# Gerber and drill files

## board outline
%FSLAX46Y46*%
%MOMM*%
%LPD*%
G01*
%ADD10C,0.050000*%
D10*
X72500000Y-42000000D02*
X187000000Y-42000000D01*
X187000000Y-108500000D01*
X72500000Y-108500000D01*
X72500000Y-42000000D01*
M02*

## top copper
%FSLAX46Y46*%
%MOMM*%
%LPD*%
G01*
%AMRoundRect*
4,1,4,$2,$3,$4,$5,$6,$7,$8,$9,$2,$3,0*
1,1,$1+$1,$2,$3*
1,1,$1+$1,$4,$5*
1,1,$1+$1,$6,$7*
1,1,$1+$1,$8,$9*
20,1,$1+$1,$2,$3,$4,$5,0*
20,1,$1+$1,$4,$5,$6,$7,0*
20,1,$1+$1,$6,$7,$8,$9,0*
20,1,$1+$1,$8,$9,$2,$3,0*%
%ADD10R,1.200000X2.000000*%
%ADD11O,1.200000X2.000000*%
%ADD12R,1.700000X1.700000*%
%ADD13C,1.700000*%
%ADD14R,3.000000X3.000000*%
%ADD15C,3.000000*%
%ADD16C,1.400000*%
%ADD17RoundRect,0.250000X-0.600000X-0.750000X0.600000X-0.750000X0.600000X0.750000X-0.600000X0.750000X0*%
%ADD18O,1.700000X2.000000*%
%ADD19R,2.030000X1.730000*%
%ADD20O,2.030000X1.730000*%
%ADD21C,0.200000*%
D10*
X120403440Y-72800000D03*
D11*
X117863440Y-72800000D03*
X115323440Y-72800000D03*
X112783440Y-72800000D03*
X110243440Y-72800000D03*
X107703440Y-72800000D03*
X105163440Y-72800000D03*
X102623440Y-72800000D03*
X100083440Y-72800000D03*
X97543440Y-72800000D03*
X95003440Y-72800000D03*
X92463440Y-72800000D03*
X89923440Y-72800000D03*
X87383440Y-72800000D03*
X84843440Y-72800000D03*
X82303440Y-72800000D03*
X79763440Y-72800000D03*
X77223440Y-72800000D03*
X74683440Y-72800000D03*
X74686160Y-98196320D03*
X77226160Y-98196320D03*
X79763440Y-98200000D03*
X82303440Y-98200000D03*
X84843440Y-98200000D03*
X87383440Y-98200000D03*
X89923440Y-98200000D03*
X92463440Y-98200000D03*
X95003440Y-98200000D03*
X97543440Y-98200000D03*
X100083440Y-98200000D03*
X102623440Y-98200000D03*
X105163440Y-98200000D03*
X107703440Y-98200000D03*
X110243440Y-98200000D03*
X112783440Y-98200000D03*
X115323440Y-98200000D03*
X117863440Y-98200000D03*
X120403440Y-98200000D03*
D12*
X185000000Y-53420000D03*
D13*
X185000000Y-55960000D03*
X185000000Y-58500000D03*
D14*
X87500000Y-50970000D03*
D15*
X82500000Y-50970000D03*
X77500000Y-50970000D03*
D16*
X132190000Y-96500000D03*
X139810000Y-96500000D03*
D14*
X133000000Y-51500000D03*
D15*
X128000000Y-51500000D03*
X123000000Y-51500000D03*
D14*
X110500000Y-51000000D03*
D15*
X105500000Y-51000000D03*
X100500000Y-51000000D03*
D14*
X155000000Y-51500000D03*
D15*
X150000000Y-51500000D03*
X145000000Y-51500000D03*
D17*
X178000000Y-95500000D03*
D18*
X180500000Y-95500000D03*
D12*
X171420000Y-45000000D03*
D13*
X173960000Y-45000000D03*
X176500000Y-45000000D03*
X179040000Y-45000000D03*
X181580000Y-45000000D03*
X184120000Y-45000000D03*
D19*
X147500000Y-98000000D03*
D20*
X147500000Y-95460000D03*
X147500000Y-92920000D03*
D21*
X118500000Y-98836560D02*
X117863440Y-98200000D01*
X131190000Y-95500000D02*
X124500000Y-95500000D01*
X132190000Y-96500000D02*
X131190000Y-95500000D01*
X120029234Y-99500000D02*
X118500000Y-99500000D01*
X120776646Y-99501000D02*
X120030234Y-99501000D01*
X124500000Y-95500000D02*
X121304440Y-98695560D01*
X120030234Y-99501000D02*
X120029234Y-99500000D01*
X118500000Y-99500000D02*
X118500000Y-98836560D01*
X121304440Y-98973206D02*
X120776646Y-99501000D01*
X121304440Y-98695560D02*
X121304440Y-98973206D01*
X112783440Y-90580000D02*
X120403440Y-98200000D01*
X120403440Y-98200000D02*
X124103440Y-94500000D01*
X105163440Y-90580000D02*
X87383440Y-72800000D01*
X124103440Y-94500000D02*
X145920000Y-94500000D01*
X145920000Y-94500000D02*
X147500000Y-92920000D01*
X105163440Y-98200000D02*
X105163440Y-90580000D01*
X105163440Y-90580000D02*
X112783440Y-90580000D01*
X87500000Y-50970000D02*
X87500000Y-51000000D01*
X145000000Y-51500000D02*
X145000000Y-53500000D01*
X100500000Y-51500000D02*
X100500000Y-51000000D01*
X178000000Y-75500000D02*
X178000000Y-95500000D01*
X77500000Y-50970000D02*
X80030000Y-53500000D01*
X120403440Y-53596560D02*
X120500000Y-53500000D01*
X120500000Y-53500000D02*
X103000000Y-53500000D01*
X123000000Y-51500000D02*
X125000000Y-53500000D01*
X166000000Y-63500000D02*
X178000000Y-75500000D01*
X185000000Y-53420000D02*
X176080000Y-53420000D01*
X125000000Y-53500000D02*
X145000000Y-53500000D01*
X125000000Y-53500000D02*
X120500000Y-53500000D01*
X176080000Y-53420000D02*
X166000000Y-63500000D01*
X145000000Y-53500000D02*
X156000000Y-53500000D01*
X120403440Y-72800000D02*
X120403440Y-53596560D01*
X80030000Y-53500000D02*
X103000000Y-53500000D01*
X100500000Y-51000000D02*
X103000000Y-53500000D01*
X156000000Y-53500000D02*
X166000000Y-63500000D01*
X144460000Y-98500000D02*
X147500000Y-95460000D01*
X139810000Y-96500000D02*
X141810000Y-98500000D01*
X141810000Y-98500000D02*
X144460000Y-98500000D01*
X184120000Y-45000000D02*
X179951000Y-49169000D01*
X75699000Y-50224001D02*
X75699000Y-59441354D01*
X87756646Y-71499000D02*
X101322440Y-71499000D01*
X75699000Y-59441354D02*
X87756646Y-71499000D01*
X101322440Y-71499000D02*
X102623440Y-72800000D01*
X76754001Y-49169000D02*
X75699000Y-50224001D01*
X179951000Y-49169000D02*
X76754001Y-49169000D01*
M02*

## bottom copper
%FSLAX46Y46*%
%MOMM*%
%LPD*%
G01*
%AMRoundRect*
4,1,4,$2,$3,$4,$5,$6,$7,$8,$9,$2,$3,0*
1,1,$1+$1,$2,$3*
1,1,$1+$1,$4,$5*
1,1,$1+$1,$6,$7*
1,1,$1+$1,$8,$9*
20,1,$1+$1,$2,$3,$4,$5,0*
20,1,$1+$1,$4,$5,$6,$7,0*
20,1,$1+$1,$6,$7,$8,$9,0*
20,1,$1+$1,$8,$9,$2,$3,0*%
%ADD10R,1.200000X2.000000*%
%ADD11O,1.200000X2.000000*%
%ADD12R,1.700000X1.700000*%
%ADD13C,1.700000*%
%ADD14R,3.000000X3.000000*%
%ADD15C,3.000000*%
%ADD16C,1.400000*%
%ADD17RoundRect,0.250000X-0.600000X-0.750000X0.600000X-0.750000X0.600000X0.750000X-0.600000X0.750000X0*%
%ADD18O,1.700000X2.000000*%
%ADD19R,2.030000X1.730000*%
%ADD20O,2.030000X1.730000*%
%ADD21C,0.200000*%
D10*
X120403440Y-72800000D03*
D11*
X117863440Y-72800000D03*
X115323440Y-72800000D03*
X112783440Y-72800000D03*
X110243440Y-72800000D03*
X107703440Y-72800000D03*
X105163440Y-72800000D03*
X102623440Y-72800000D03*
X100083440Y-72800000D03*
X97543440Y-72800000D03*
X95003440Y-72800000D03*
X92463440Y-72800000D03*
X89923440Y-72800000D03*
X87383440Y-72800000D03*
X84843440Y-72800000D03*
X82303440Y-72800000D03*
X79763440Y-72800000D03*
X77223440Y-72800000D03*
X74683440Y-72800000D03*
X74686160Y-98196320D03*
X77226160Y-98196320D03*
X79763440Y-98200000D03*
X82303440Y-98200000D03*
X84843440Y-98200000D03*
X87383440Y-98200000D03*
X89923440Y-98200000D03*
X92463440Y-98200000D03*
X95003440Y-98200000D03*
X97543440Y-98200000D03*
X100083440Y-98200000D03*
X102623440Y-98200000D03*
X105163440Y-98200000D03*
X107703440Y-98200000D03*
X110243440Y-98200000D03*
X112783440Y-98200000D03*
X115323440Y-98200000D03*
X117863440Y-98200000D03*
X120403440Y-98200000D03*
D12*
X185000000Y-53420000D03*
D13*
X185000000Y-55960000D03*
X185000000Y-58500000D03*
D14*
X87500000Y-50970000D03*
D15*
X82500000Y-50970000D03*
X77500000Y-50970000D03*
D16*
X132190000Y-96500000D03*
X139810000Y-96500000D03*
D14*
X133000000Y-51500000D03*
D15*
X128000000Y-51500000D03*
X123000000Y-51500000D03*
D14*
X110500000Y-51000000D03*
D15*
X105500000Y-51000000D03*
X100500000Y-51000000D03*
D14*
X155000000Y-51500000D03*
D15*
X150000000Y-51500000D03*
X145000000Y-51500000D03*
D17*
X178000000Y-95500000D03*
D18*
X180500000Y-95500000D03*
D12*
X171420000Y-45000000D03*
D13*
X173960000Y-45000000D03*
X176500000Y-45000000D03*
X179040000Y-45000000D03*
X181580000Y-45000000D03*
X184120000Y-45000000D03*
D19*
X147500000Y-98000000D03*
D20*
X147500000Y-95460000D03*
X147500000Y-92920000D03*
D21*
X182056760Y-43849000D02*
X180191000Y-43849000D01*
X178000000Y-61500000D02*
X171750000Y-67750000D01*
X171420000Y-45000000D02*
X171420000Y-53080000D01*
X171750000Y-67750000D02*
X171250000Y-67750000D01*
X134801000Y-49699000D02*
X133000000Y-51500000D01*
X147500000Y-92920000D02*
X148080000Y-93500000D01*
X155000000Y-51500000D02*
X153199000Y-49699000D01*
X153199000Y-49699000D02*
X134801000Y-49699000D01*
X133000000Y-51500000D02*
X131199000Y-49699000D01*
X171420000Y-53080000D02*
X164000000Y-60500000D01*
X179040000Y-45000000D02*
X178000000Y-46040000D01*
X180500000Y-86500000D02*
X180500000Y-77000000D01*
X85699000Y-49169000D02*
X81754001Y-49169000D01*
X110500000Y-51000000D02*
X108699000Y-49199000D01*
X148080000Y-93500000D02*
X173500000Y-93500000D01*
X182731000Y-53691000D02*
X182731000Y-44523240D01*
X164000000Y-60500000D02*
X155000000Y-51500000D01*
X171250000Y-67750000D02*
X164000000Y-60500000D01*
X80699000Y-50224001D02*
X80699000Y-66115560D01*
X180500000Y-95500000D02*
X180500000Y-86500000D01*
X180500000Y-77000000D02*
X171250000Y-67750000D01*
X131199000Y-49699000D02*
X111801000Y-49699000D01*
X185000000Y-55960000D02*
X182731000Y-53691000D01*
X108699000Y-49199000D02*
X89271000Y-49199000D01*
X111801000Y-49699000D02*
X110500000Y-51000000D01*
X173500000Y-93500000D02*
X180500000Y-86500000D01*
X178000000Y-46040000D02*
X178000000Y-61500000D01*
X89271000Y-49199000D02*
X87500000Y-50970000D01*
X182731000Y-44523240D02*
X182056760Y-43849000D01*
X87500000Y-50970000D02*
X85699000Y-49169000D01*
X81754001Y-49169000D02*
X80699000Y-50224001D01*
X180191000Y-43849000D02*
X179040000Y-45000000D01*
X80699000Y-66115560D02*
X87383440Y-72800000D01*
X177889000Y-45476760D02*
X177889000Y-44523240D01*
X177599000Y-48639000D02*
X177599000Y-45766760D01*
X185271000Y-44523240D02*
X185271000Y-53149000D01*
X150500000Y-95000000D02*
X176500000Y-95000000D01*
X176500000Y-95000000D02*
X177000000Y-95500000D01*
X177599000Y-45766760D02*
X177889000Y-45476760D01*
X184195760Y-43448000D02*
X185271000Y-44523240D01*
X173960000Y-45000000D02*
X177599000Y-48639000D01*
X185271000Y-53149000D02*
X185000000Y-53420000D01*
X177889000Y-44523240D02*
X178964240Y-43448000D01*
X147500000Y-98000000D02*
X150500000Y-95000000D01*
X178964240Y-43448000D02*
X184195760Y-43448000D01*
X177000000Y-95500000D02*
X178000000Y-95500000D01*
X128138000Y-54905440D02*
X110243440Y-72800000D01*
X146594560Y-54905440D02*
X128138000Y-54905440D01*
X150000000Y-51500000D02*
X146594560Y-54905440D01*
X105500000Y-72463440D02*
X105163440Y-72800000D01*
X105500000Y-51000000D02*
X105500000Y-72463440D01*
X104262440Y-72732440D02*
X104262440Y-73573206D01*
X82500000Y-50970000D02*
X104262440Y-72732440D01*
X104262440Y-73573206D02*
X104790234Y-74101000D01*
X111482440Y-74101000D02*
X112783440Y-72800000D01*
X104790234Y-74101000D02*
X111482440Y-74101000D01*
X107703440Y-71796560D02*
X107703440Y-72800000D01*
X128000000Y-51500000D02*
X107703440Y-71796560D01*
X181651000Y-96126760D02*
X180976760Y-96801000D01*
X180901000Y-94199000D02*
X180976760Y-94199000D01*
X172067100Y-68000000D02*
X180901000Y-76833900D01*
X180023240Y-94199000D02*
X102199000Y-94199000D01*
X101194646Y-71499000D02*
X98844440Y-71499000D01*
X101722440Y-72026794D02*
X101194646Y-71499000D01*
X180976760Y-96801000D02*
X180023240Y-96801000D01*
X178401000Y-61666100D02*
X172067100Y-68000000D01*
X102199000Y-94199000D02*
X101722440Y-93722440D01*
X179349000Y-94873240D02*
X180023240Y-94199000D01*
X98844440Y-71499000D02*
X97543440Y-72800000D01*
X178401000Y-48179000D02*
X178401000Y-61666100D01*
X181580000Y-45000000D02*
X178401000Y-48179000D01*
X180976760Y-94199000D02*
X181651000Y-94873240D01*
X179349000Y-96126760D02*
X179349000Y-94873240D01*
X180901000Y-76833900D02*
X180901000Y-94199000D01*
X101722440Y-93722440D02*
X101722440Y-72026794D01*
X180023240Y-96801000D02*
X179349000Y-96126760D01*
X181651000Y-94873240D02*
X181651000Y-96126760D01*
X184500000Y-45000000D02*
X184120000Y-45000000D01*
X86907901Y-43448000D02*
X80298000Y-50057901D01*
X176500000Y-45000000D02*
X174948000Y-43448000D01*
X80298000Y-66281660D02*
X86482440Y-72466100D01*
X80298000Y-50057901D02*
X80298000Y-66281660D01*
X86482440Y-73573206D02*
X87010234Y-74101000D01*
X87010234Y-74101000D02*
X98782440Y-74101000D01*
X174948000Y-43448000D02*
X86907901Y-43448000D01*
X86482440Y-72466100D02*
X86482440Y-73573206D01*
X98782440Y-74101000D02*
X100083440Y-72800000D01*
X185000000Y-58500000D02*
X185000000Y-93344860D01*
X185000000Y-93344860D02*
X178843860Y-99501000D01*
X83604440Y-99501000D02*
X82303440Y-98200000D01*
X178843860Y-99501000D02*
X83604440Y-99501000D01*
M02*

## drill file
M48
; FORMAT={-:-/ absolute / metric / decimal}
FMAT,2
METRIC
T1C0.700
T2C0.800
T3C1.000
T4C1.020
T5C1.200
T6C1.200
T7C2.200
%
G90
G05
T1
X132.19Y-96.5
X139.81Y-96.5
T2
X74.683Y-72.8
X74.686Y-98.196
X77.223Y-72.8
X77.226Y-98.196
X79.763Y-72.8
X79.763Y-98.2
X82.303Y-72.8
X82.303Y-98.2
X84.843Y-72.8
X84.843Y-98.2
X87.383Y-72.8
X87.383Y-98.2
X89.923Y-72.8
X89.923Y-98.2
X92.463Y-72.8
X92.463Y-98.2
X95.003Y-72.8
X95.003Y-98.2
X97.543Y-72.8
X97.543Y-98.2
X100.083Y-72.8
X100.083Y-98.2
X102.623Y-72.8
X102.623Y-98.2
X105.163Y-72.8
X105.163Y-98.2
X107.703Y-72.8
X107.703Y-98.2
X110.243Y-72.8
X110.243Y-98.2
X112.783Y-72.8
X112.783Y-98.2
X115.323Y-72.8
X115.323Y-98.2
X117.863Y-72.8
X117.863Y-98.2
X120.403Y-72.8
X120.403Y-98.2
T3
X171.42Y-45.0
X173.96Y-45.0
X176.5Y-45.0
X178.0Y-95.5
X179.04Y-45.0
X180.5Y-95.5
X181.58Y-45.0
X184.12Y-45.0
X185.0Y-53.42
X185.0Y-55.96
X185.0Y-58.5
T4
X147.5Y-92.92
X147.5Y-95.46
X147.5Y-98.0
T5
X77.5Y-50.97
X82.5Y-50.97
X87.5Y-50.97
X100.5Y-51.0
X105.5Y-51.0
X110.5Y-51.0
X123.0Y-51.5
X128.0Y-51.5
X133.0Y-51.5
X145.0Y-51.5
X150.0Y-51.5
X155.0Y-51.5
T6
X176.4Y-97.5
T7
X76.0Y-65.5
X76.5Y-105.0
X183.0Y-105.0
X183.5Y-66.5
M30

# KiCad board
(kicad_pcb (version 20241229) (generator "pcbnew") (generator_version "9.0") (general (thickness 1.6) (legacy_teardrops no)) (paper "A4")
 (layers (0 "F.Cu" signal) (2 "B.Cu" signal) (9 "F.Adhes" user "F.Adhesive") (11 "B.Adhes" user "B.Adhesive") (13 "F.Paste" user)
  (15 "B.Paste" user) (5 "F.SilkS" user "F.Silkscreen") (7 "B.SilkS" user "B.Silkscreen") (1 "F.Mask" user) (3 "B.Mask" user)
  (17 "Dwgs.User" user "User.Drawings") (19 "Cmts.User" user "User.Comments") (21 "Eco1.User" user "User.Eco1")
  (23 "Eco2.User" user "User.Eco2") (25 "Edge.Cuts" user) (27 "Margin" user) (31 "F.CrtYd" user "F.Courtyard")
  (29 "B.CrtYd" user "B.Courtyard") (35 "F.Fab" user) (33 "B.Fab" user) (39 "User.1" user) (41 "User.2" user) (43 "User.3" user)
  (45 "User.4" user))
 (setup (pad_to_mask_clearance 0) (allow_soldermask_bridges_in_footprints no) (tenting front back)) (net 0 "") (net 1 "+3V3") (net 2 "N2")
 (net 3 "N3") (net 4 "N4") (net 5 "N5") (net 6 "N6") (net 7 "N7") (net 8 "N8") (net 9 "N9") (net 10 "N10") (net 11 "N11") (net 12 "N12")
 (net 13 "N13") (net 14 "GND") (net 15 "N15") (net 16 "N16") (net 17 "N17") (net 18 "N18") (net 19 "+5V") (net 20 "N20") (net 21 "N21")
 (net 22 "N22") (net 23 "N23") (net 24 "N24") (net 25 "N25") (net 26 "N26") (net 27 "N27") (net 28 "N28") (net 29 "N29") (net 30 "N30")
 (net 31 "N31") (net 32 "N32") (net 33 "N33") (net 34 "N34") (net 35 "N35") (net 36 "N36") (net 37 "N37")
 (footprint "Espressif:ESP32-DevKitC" (layer "F.Cu") (at 120.40344 72.8 -90)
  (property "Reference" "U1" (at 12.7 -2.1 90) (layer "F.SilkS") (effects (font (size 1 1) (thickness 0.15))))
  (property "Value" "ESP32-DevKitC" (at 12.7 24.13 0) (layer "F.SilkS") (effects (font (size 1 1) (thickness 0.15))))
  (pad "1" thru_hole rect (at 0 0 180) (size 1.2 2) (drill 0.8) (layers "*.Cu" "*.Mask") (remove_unused_layers no) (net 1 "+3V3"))
  (pad "2" thru_hole oval (at 0 2.54 180) (size 1.2 2) (drill 0.8) (layers "*.Cu" "*.Mask") (remove_unused_layers no) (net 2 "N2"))
  (pad "3" thru_hole oval (at 0 5.08 180) (size 1.2 2) (drill 0.8) (layers "*.Cu" "*.Mask") (remove_unused_layers no) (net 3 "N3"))
  (pad "4" thru_hole oval (at 0 7.62 180) (size 1.2 2) (drill 0.8) (layers "*.Cu" "*.Mask") (remove_unused_layers no) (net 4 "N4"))
  (pad "5" thru_hole oval (at 0 10.16 180) (size 1.2 2) (drill 0.8) (layers "*.Cu" "*.Mask") (remove_unused_layers no) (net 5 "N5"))
  (pad "6" thru_hole oval (at 0 12.7 180) (size 1.2 2) (drill 0.8) (layers "*.Cu" "*.Mask") (remove_unused_layers no) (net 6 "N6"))
  (pad "7" thru_hole oval (at 0 15.24 180) (size 1.2 2) (drill 0.8) (layers "*.Cu" "*.Mask") (remove_unused_layers no) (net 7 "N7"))
  (pad "8" thru_hole oval (at 0 17.78 180) (size 1.2 2) (drill 0.8) (layers "*.Cu" "*.Mask") (remove_unused_layers no) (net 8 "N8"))
  (pad "9" thru_hole oval (at 0 20.32 180) (size 1.2 2) (drill 0.8) (layers "*.Cu" "*.Mask") (remove_unused_layers no) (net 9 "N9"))
  (pad "10" thru_hole oval (at 0 22.86 180) (size 1.2 2) (drill 0.8) (layers "*.Cu" "*.Mask") (remove_unused_layers no) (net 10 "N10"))
  (pad "11" thru_hole oval (at 0 25.4 180) (size 1.2 2) (drill 0.8) (layers "*.Cu" "*.Mask") (remove_unused_layers no) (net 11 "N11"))
  (pad "12" thru_hole oval (at 0 27.94 180) (size 1.2 2) (drill 0.8) (layers "*.Cu" "*.Mask") (remove_unused_layers no) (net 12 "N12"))
  (pad "13" thru_hole oval (at 0 30.48 180) (size 1.2 2) (drill 0.8) (layers "*.Cu" "*.Mask") (remove_unused_layers no) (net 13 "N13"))
  (pad "14" thru_hole oval (at 0 33.02 180) (size 1.2 2) (drill 0.8) (layers "*.Cu" "*.Mask") (remove_unused_layers no) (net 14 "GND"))
  (pad "15" thru_hole oval (at 0 35.56 180) (size 1.2 2) (drill 0.8) (layers "*.Cu" "*.Mask") (remove_unused_layers no) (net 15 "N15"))
  (pad "16" thru_hole oval (at 0 38.1 180) (size 1.2 2) (drill 0.8) (layers "*.Cu" "*.Mask") (remove_unused_layers no) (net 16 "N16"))
  (pad "17" thru_hole oval (at 0 40.64 180) (size 1.2 2) (drill 0.8) (layers "*.Cu" "*.Mask") (remove_unused_layers no) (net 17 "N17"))
  (pad "18" thru_hole oval (at 0 43.18 180) (size 1.2 2) (drill 0.8) (layers "*.Cu" "*.Mask") (remove_unused_layers no) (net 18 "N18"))
  (pad "19" thru_hole oval (at 0 45.72 180) (size 1.2 2) (drill 0.8) (layers "*.Cu" "*.Mask") (remove_unused_layers no) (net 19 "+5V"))
  (pad "20" thru_hole oval (at 25.39632 45.71728 180) (size 1.2 2) (drill 0.8) (layers "*.Cu" "*.Mask") (remove_unused_layers no)
   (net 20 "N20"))
  (pad "21" thru_hole oval (at 25.39632 43.17728 180) (size 1.2 2) (drill 0.8) (layers "*.Cu" "*.Mask") (remove_unused_layers no)
   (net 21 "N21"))
  (pad "22" thru_hole oval (at 25.4 40.64 180) (size 1.2 2) (drill 0.8) (layers "*.Cu" "*.Mask") (remove_unused_layers no) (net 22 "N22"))
  (pad "23" thru_hole oval (at 25.4 38.1 180) (size 1.2 2) (drill 0.8) (layers "*.Cu" "*.Mask") (remove_unused_layers no) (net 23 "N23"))
  (pad "24" thru_hole oval (at 25.4 35.56 180) (size 1.2 2) (drill 0.8) (layers "*.Cu" "*.Mask") (remove_unused_layers no) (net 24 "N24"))
  (pad "25" thru_hole oval (at 25.4 33.02 180) (size 1.2 2) (drill 0.8) (layers "*.Cu" "*.Mask") (remove_unused_layers no) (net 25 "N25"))
  (pad "26" thru_hole oval (at 25.4 30.48 180) (size 1.2 2) (drill 0.8) (layers "*.Cu" "*.Mask") (remove_unused_layers no) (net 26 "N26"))
  (pad "27" thru_hole oval (at 25.4 27.94 180) (size 1.2 2) (drill 0.8) (layers "*.Cu" "*.Mask") (remove_unused_layers no) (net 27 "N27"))
  (pad "28" thru_hole oval (at 25.4 25.4 180) (size 1.2 2) (drill 0.8) (layers "*.Cu" "*.Mask") (remove_unused_layers no) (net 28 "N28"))
  (pad "29" thru_hole oval (at 25.4 22.86 180) (size 1.2 2) (drill 0.8) (layers "*.Cu" "*.Mask") (remove_unused_layers no) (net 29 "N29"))
  (pad "30" thru_hole oval (at 25.4 20.32 180) (size 1.2 2) (drill 0.8) (layers "*.Cu" "*.Mask") (remove_unused_layers no) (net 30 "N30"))
  (pad "31" thru_hole oval (at 25.4 17.78 180) (size 1.2 2) (drill 0.8) (layers "*.Cu" "*.Mask") (remove_unused_layers no) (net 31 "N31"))
  (pad "32" thru_hole oval (at 25.4 15.24 180) (size 1.2 2) (drill 0.8) (layers "*.Cu" "*.Mask") (remove_unused_layers no) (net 14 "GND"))
  (pad "33" thru_hole oval (at 25.4 12.7 180) (size 1.2 2) (drill 0.8) (layers "*.Cu" "*.Mask") (remove_unused_layers no) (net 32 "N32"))
  (pad "34" thru_hole oval (at 25.4 10.16 180) (size 1.2 2) (drill 0.8) (layers "*.Cu" "*.Mask") (remove_unused_layers no) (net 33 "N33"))
  (pad "35" thru_hole oval (at 25.4 7.62 180) (size 1.2 2) (drill 0.8) (layers "*.Cu" "*.Mask") (remove_unused_layers no) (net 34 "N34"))
  (pad "36" thru_hole oval (at 25.4 5.08 180) (size 1.2 2) (drill 0.8) (layers "*.Cu" "*.Mask") (remove_unused_layers no) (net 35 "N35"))
  (pad "37" thru_hole oval (at 25.4 2.54 180) (size 1.2 2) (drill 0.8) (layers "*.Cu" "*.Mask") (remove_unused_layers no) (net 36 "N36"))
  (pad "38" thru_hole oval (at 25.4 0 180) (size 1.2 2) (drill 0.8) (layers "*.Cu" "*.Mask") (remove_unused_layers no) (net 14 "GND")))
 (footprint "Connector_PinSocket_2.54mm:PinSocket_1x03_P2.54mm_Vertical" (layer "F.Cu") (at 185 53.42)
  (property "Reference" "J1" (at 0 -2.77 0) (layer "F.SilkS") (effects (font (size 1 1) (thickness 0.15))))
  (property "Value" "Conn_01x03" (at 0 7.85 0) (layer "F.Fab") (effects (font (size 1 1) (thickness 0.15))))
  (pad "1" thru_hole rect (at 0 0) (size 1.7 1.7) (drill 1) (layers "*.Cu" "*.Mask") (remove_unused_layers no) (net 1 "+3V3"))
  (pad "2" thru_hole circle (at 0 2.54) (size 1.7 1.7) (drill 1) (layers "*.Cu" "*.Mask") (remove_unused_layers no) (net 14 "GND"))
  (pad "3" thru_hole circle (at 0 5.08) (size 1.7 1.7) (drill 1) (layers "*.Cu" "*.Mask") (remove_unused_layers no) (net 23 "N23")))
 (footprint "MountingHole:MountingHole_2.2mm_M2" (layer "F.Cu") (at 76.5 105)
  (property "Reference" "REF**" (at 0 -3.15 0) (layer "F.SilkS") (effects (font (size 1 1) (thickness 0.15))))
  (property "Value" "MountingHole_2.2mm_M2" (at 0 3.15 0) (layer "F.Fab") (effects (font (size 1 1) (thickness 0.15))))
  (pad "" np_thru_hole circle (at 0 0) (size 2.2 2.2) (drill 2.2) (layers "*.Cu" "*.Mask")))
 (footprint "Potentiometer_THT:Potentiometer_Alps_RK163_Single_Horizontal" (layer "F.Cu") (at 87.5 50.97 -90)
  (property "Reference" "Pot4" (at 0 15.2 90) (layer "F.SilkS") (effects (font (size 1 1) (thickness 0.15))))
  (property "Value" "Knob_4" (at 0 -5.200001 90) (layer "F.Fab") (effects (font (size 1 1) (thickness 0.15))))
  (pad "1" thru_hole rect (at 0 0 90) (size 3 3) (drill 1.2) (layers "*.Cu" "*.Mask") (remove_unused_layers no) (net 14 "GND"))
  (pad "2" thru_hole circle (at 0 5 90) (size 3 3) (drill 1.2) (layers "*.Cu" "*.Mask") (remove_unused_layers no) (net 4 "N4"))
  (pad "3" thru_hole circle (at 0 10 90) (size 3 3) (drill 1.2) (layers "*.Cu" "*.Mask") (remove_unused_layers no) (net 1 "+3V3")))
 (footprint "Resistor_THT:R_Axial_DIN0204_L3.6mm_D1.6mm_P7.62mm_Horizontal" (layer "F.Cu") (at 132.19 96.5)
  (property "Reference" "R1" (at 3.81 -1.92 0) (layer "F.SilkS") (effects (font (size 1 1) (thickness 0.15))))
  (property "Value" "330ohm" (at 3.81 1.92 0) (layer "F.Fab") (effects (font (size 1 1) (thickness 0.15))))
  (pad "1" thru_hole circle (at 0 0) (size 1.4 1.4) (drill 0.7) (layers "*.Cu" "*.Mask") (remove_unused_layers no) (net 36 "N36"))
  (pad "2" thru_hole circle (at 7.62 0) (size 1.4 1.4) (drill 0.7) (layers "*.Cu" "*.Mask") (remove_unused_layers no) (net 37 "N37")))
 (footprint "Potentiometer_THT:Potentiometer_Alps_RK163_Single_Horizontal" (layer "F.Cu") (at 133 51.5 -90)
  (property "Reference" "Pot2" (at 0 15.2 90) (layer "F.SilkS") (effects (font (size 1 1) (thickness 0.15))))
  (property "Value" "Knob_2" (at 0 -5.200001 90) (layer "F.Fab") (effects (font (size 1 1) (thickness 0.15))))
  (pad "1" thru_hole rect (at 0 0 90) (size 3 3) (drill 1.2) (layers "*.Cu" "*.Mask") (remove_unused_layers no) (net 14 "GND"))
  (pad "2" thru_hole circle (at 0 5 90) (size 3 3) (drill 1.2) (layers "*.Cu" "*.Mask") (remove_unused_layers no) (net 6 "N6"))
  (pad "3" thru_hole circle (at 0 10 90) (size 3 3) (drill 1.2) (layers "*.Cu" "*.Mask") (remove_unused_layers no) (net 1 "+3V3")))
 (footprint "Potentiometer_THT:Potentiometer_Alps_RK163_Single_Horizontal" (layer "F.Cu") (at 110.5 51 -90)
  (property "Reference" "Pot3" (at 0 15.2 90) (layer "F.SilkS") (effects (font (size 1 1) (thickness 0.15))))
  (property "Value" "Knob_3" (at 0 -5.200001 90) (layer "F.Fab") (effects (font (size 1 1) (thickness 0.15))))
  (pad "1" thru_hole rect (at 0 0 90) (size 3 3) (drill 1.2) (layers "*.Cu" "*.Mask") (remove_unused_layers no) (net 14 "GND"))
  (pad "2" thru_hole circle (at 0 5 90) (size 3 3) (drill 1.2) (layers "*.Cu" "*.Mask") (remove_unused_layers no) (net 7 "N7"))
  (pad "3" thru_hole circle (at 0 10 90) (size 3 3) (drill 1.2) (layers "*.Cu" "*.Mask") (remove_unused_layers no) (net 1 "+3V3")))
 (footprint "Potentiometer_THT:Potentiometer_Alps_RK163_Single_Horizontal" (layer "F.Cu") (at 155 51.5 -90)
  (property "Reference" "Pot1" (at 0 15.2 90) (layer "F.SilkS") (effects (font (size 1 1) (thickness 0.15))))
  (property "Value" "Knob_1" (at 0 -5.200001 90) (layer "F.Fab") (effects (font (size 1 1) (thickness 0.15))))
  (pad "1" thru_hole rect (at 0 0 90) (size 3 3) (drill 1.2) (layers "*.Cu" "*.Mask") (remove_unused_layers no) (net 14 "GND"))
  (pad "2" thru_hole circle (at 0 5 90) (size 3 3) (drill 1.2) (layers "*.Cu" "*.Mask") (remove_unused_layers no) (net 5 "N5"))
  (pad "3" thru_hole circle (at 0 10 90) (size 3 3) (drill 1.2) (layers "*.Cu" "*.Mask") (remove_unused_layers no) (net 1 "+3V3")))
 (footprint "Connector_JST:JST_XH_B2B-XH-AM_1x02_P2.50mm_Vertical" (layer "F.Cu") (at 178 95.5)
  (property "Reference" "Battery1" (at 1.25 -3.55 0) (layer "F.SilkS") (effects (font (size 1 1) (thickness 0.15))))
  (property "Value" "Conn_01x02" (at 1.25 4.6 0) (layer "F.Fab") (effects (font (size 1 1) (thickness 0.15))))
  (pad "" np_thru_hole circle (at -1.6 2) (size 1.2 1.2) (drill 1.2) (layers "*.Cu" "*.Mask"))
  (pad "1" thru_hole roundrect (at 0 0) (size 1.7 2) (drill 1) (layers "*.Cu" "*.Mask") (remove_unused_layers no)
   (roundrect_rratio 0.147059) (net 1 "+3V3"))
  (pad "2" thru_hole oval (at 2.5 0) (size 1.7 2) (drill 1) (layers "*.Cu" "*.Mask") (remove_unused_layers no) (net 14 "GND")))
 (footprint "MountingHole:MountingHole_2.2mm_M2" (layer "F.Cu") (at 76 65.5)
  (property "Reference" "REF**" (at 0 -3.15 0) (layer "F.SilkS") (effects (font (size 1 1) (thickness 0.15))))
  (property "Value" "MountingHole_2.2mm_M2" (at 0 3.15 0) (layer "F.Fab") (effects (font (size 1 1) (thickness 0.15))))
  (pad "" np_thru_hole circle (at 0 0) (size 2.2 2.2) (drill 2.2) (layers "*.Cu" "*.Mask")))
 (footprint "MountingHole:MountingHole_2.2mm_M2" (layer "F.Cu") (at 183.5 66.5)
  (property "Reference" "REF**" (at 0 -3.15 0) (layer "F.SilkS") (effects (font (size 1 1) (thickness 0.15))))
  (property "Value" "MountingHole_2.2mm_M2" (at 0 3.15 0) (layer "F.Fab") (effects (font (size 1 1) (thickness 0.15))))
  (pad "" np_thru_hole circle (at 0 0) (size 2.2 2.2) (drill 2.2) (layers "*.Cu" "*.Mask")))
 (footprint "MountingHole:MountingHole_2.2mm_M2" (layer "F.Cu") (at 183 105)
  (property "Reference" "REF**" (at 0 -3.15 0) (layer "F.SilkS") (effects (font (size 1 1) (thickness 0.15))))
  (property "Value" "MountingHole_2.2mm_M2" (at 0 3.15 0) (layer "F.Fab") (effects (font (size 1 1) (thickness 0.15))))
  (pad "" np_thru_hole circle (at 0 0) (size 2.2 2.2) (drill 2.2) (layers "*.Cu" "*.Mask")))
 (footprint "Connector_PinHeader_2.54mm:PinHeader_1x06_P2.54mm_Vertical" (layer "B.Cu") (at 171.42 45 -90)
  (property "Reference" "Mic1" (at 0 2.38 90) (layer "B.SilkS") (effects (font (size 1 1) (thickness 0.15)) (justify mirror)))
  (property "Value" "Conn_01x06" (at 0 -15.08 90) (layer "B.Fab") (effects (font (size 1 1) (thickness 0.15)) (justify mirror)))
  (pad "1" thru_hole rect (at 0 0 270) (size 1.7 1.7) (drill 1) (layers "*.Cu" "*.Mask") (remove_unused_layers no) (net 14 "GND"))
  (pad "2" thru_hole circle (at 0 -2.54 270) (size 1.7 1.7) (drill 1) (layers "*.Cu" "*.Mask") (remove_unused_layers no) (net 1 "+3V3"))
  (pad "3" thru_hole circle (at 0 -5.08 270) (size 1.7 1.7) (drill 1) (layers "*.Cu" "*.Mask") (remove_unused_layers no) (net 9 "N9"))
  (pad "4" thru_hole circle (at 0 -7.62 270) (size 1.7 1.7) (drill 1) (layers "*.Cu" "*.Mask") (remove_unused_layers no) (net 14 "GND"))
  (pad "5" thru_hole circle (at 0 -10.16 270) (size 1.7 1.7) (drill 1) (layers "*.Cu" "*.Mask") (remove_unused_layers no) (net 10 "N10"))
  (pad "6" thru_hole circle (at 0 -12.7 270) (size 1.7 1.7) (drill 1) (layers "*.Cu" "*.Mask") (remove_unused_layers no) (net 8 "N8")))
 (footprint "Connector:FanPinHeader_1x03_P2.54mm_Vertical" (layer "B.Cu") (at 147.5 98 90)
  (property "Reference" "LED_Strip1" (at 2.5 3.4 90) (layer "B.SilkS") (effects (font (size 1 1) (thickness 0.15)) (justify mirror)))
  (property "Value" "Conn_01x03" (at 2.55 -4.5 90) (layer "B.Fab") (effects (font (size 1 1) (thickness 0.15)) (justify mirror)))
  (pad "1" thru_hole rect (at 0 0) (size 2.03 1.73) (drill 1.02) (layers "*.Cu" "*.Mask") (remove_unused_layers no) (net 1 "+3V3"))
  (pad "2" thru_hole oval (at 2.54 0) (size 2.03 1.73) (drill 1.02) (layers "*.Cu" "*.Mask") (remove_unused_layers no) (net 37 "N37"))
  (pad "3" thru_hole oval (at 5.08 0) (size 2.03 1.73) (drill 1.02) (layers "*.Cu" "*.Mask") (remove_unused_layers no) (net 14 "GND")))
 (gr_rect (start 72.5 42) (end 187 108.5) (stroke (width 0.05) (type default)) (fill no) (layer "Edge.Cuts"))
 (segment (start 118.5 98.83656) (end 117.86344 98.2) (width 0.2) (layer "F.Cu") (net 36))
 (segment (start 131.19 95.5) (end 124.5 95.5) (width 0.2) (layer "F.Cu") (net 36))
 (segment (start 132.19 96.5) (end 131.19 95.5) (width 0.2) (layer "F.Cu") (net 36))
 (segment (start 120.029234 99.5) (end 118.5 99.5) (width 0.2) (layer "F.Cu") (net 36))
 (segment (start 120.776646 99.501) (end 120.030234 99.501) (width 0.2) (layer "F.Cu") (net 36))
 (segment (start 124.5 95.5) (end 121.30444 98.69556) (width 0.2) (layer "F.Cu") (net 36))
 (segment (start 120.030234 99.501) (end 120.029234 99.5) (width 0.2) (layer "F.Cu") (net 36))
 (segment (start 118.5 99.5) (end 118.5 98.83656) (width 0.2) (layer "F.Cu") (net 36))
 (segment (start 121.30444 98.973206) (end 120.776646 99.501) (width 0.2) (layer "F.Cu") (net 36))
 (segment (start 121.30444 98.69556) (end 121.30444 98.973206) (width 0.2) (layer "F.Cu") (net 36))
 (segment (start 112.78344 90.58) (end 120.40344 98.2) (width 0.2) (layer "F.Cu") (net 14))
 (segment (start 120.40344 98.2) (end 124.10344 94.5) (width 0.2) (layer "F.Cu") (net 14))
 (segment (start 105.16344 90.58) (end 87.38344 72.8) (width 0.2) (layer "F.Cu") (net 14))
 (segment (start 124.10344 94.5) (end 145.92 94.5) (width 0.2) (layer "F.Cu") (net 14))
 (segment (start 145.92 94.5) (end 147.5 92.92) (width 0.2) (layer "F.Cu") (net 14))
 (segment (start 105.16344 98.2) (end 105.16344 90.58) (width 0.2) (layer "F.Cu") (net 14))
 (segment (start 105.16344 90.58) (end 112.78344 90.58) (width 0.2) (layer "F.Cu") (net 14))
 (segment (start 87.5 50.97) (end 87.5 51) (width 0.2) (layer "F.Cu") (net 14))
 (segment (start 182.05676 43.849) (end 180.191 43.849) (width 0.2) (layer "B.Cu") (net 14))
 (segment (start 178 61.5) (end 171.75 67.75) (width 0.2) (layer "B.Cu") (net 14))
 (segment (start 171.42 45) (end 171.42 53.08) (width 0.2) (layer "B.Cu") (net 14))
 (segment (start 171.75 67.75) (end 171.25 67.75) (width 0.2) (layer "B.Cu") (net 14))
 (segment (start 134.801 49.699) (end 133 51.5) (width 0.2) (layer "B.Cu") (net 14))
 (segment (start 147.5 92.92) (end 148.08 93.5) (width 0.2) (layer "B.Cu") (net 14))
 (segment (start 155 51.5) (end 153.199 49.699) (width 0.2) (layer "B.Cu") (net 14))
 (segment (start 153.199 49.699) (end 134.801 49.699) (width 0.2) (layer "B.Cu") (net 14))
 (segment (start 133 51.5) (end 131.199 49.699) (width 0.2) (layer "B.Cu") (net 14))
 (segment (start 171.42 53.08) (end 164 60.5) (width 0.2) (layer "B.Cu") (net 14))
 (segment (start 179.04 45) (end 178 46.04) (width 0.2) (layer "B.Cu") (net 14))
 (segment (start 180.5 86.5) (end 180.5 77) (width 0.2) (layer "B.Cu") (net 14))
 (segment (start 85.699 49.169) (end 81.754001 49.169) (width 0.2) (layer "B.Cu") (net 14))
 (segment (start 110.5 51) (end 108.699 49.199) (width 0.2) (layer "B.Cu") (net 14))
 (segment (start 148.08 93.5) (end 173.5 93.5) (width 0.2) (layer "B.Cu") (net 14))
 (segment (start 182.731 53.691) (end 182.731 44.52324) (width 0.2) (layer "B.Cu") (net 14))
 (segment (start 164 60.5) (end 155 51.5) (width 0.2) (layer "B.Cu") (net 14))
 (segment (start 171.25 67.75) (end 164 60.5) (width 0.2) (layer "B.Cu") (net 14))
 (segment (start 80.699 50.224001) (end 80.699 66.11556) (width 0.2) (layer "B.Cu") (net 14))
 (segment (start 180.5 95.5) (end 180.5 86.5) (width 0.2) (layer "B.Cu") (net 14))
 (segment (start 180.5 77) (end 171.25 67.75) (width 0.2) (layer "B.Cu") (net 14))
 (segment (start 131.199 49.699) (end 111.801 49.699) (width 0.2) (layer "B.Cu") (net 14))
 (segment (start 185 55.96) (end 182.731 53.691) (width 0.2) (layer "B.Cu") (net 14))
 (segment (start 108.699 49.199) (end 89.271 49.199) (width 0.2) (layer "B.Cu") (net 14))
 (segment (start 111.801 49.699) (end 110.5 51) (width 0.2) (layer "B.Cu") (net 14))
 (segment (start 173.5 93.5) (end 180.5 86.5) (width 0.2) (layer "B.Cu") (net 14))
 (segment (start 178 46.04) (end 178 61.5) (width 0.2) (layer "B.Cu") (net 14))
 (segment (start 89.271 49.199) (end 87.5 50.97) (width 0.2) (layer "B.Cu") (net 14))
 (segment (start 182.731 44.52324) (end 182.05676 43.849) (width 0.2) (layer "B.Cu") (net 14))
 (segment (start 87.5 50.97) (end 85.699 49.169) (width 0.2) (layer "B.Cu") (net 14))
 (segment (start 81.754001 49.169) (end 80.699 50.224001) (width 0.2) (layer "B.Cu") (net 14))
 (segment (start 180.191 43.849) (end 179.04 45) (width 0.2) (layer "B.Cu") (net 14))
 (segment (start 80.699 66.11556) (end 87.38344 72.8) (width 0.2) (layer "B.Cu") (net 14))
 (segment (start 145 51.5) (end 145 53.5) (width 0.2) (layer "F.Cu") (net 1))
 (segment (start 100.5 51.5) (end 100.5 51) (width 0.2) (layer "F.Cu") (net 1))
 (segment (start 178 75.5) (end 178 95.5) (width 0.2) (layer "F.Cu") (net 1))
 (segment (start 77.5 50.97) (end 80.03 53.5) (width 0.2) (layer "F.Cu") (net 1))
 (segment (start 120.40344 53.59656) (end 120.5 53.5) (width 0.2) (layer "F.Cu") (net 1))
 (segment (start 120.5 53.5) (end 103 53.5) (width 0.2) (layer "F.Cu") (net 1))
 (segment (start 123 51.5) (end 125 53.5) (width 0.2) (layer "F.Cu") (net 1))
 (segment (start 166 63.5) (end 178 75.5) (width 0.2) (layer "F.Cu") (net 1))
 (segment (start 185 53.42) (end 176.08 53.42) (width 0.2) (layer "F.Cu") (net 1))
 (segment (start 125 53.5) (end 145 53.5) (width 0.2) (layer "F.Cu") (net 1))
 (segment (start 125 53.5) (end 120.5 53.5) (width 0.2) (layer "F.Cu") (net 1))
 (segment (start 176.08 53.42) (end 166 63.5) (width 0.2) (layer "F.Cu") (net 1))
 (segment (start 145 53.5) (end 156 53.5) (width 0.2) (layer "F.Cu") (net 1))
 (segment (start 120.40344 72.8) (end 120.40344 53.59656) (width 0.2) (layer "F.Cu") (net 1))
 (segment (start 80.03 53.5) (end 103 53.5) (width 0.2) (layer "F.Cu") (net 1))
 (segment (start 100.5 51) (end 103 53.5) (width 0.2) (layer "F.Cu") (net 1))
 (segment (start 156 53.5) (end 166 63.5) (width 0.2) (layer "F.Cu") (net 1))
 (segment (start 177.889 45.47676) (end 177.889 44.52324) (width 0.2) (layer "B.Cu") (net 1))
 (segment (start 177.599 48.639) (end 177.599 45.76676) (width 0.2) (layer "B.Cu") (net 1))
 (segment (start 185.271 44.52324) (end 185.271 53.149) (width 0.2) (layer "B.Cu") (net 1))
 (segment (start 150.5 95) (end 176.5 95) (width 0.2) (layer "B.Cu") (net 1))
 (segment (start 176.5 95) (end 177 95.5) (width 0.2) (layer "B.Cu") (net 1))
 (segment (start 177.599 45.76676) (end 177.889 45.47676) (width 0.2) (layer "B.Cu") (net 1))
 (segment (start 184.19576 43.448) (end 185.271 44.52324) (width 0.2) (layer "B.Cu") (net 1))
 (segment (start 173.96 45) (end 177.599 48.639) (width 0.2) (layer "B.Cu") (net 1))
 (segment (start 185.271 53.149) (end 185 53.42) (width 0.2) (layer "B.Cu") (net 1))
 (segment (start 177.889 44.52324) (end 178.96424 43.448) (width 0.2) (layer "B.Cu") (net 1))
 (segment (start 147.5 98) (end 150.5 95) (width 0.2) (layer "B.Cu") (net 1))
 (segment (start 178.96424 43.448) (end 184.19576 43.448) (width 0.2) (layer "B.Cu") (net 1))
 (segment (start 177 95.5) (end 178 95.5) (width 0.2) (layer "B.Cu") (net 1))
 (segment (start 128.138 54.90544) (end 110.24344 72.8) (width 0.2) (layer "B.Cu") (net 5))
 (segment (start 146.59456 54.90544) (end 128.138 54.90544) (width 0.2) (layer "B.Cu") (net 5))
 (segment (start 150 51.5) (end 146.59456 54.90544) (width 0.2) (layer "B.Cu") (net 5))
 (segment (start 105.5 72.46344) (end 105.16344 72.8) (width 0.2) (layer "B.Cu") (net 7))
 (segment (start 105.5 51) (end 105.5 72.46344) (width 0.2) (layer "B.Cu") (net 7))
 (segment (start 104.26244 72.73244) (end 104.26244 73.573206) (width 0.2) (layer "B.Cu") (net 4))
 (segment (start 82.5 50.97) (end 104.26244 72.73244) (width 0.2) (layer "B.Cu") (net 4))
 (segment (start 104.26244 73.573206) (end 104.790234 74.101) (width 0.2) (layer "B.Cu") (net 4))
 (segment (start 111.48244 74.101) (end 112.78344 72.8) (width 0.2) (layer "B.Cu") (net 4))
 (segment (start 104.790234 74.101) (end 111.48244 74.101) (width 0.2) (layer "B.Cu") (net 4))
 (segment (start 107.70344 71.79656) (end 107.70344 72.8) (width 0.2) (layer "B.Cu") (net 6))
 (segment (start 128 51.5) (end 107.70344 71.79656) (width 0.2) (layer "B.Cu") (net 6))
 (segment (start 144.46 98.5) (end 147.5 95.46) (width 0.2) (layer "F.Cu") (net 37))
 (segment (start 139.81 96.5) (end 141.81 98.5) (width 0.2) (layer "F.Cu") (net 37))
 (segment (start 141.81 98.5) (end 144.46 98.5) (width 0.2) (layer "F.Cu") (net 37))
 (segment (start 181.651 96.12676) (end 180.97676 96.801) (width 0.2) (layer "B.Cu") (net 10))
 (segment (start 180.901 94.199) (end 180.97676 94.199) (width 0.2) (layer "B.Cu") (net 10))
 (segment (start 172.0671 68) (end 180.901 76.8339) (width 0.2) (layer "B.Cu") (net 10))
 (segment (start 180.02324 94.199) (end 102.199 94.199) (width 0.2) (layer "B.Cu") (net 10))
 (segment (start 101.194646 71.499) (end 98.84444 71.499) (width 0.2) (layer "B.Cu") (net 10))
 (segment (start 101.72244 72.026794) (end 101.194646 71.499) (width 0.2) (layer "B.Cu") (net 10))
 (segment (start 180.97676 96.801) (end 180.02324 96.801) (width 0.2) (layer "B.Cu") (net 10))
 (segment (start 178.401 61.6661) (end 172.0671 68) (width 0.2) (layer "B.Cu") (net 10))
 (segment (start 102.199 94.199) (end 101.72244 93.72244) (width 0.2) (layer "B.Cu") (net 10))
 (segment (start 179.349 94.87324) (end 180.02324 94.199) (width 0.2) (layer "B.Cu") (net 10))
 (segment (start 98.84444 71.499) (end 97.54344 72.8) (width 0.2) (layer "B.Cu") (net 10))
 (segment (start 178.401 48.179) (end 178.401 61.6661) (width 0.2) (layer "B.Cu") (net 10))
 (segment (start 181.58 45) (end 178.401 48.179) (width 0.2) (layer "B.Cu") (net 10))
 (segment (start 180.97676 94.199) (end 181.651 94.87324) (width 0.2) (layer "B.Cu") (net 10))
 (segment (start 179.349 96.12676) (end 179.349 94.87324) (width 0.2) (layer "B.Cu") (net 10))
 (segment (start 180.901 76.8339) (end 180.901 94.199) (width 0.2) (layer "B.Cu") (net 10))
 (segment (start 101.72244 93.72244) (end 101.72244 72.026794) (width 0.2) (layer "B.Cu") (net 10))
 (segment (start 180.02324 96.801) (end 179.349 96.12676) (width 0.2) (layer "B.Cu") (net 10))
 (segment (start 181.651 94.87324) (end 181.651 96.12676) (width 0.2) (layer "B.Cu") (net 10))
 (segment (start 184.12 45) (end 179.951 49.169) (width 0.2) (layer "F.Cu") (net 8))
 (segment (start 75.699 50.224001) (end 75.699 59.441354) (width 0.2) (layer "F.Cu") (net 8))
 (segment (start 87.756646 71.499) (end 101.32244 71.499) (width 0.2) (layer "F.Cu") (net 8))
 (segment (start 75.699 59.441354) (end 87.756646 71.499) (width 0.2) (layer "F.Cu") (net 8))
 (segment (start 101.32244 71.499) (end 102.62344 72.8) (width 0.2) (layer "F.Cu") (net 8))
 (segment (start 76.754001 49.169) (end 75.699 50.224001) (width 0.2) (layer "F.Cu") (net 8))
 (segment (start 179.951 49.169) (end 76.754001 49.169) (width 0.2) (layer "F.Cu") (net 8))
 (segment (start 184.5 45) (end 184.12 45) (width 0.2) (layer "B.Cu") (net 8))
 (segment (start 86.907901 43.448) (end 80.298 50.057901) (width 0.2) (layer "B.Cu") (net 9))
 (segment (start 176.5 45) (end 174.948 43.448) (width 0.2) (layer "B.Cu") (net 9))
 (segment (start 80.298 66.28166) (end 86.48244 72.4661) (width 0.2) (layer "B.Cu") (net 9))
 (segment (start 80.298 50.057901) (end 80.298 66.28166) (width 0.2) (layer "B.Cu") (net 9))
 (segment (start 86.48244 73.573206) (end 87.010234 74.101) (width 0.2) (layer "B.Cu") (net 9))
 (segment (start 87.010234 74.101) (end 98.78244 74.101) (width 0.2) (layer "B.Cu") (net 9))
 (segment (start 174.948 43.448) (end 86.907901 43.448) (width 0.2) (layer "B.Cu") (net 9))
 (segment (start 86.48244 72.4661) (end 86.48244 73.573206) (width 0.2) (layer "B.Cu") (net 9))
 (segment (start 98.78244 74.101) (end 100.08344 72.8) (width 0.2) (layer "B.Cu") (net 9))
 (segment (start 185 58.5) (end 185 93.34486) (width 0.2) (layer "B.Cu") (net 23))
 (segment (start 185 93.34486) (end 178.84386 99.501) (width 0.2) (layer "B.Cu") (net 23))
 (segment (start 83.60444 99.501) (end 82.30344 98.2) (width 0.2) (layer "B.Cu") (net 23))
 (segment (start 178.84386 99.501) (end 83.60444 99.501) (width 0.2) (layer "B.Cu") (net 23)))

